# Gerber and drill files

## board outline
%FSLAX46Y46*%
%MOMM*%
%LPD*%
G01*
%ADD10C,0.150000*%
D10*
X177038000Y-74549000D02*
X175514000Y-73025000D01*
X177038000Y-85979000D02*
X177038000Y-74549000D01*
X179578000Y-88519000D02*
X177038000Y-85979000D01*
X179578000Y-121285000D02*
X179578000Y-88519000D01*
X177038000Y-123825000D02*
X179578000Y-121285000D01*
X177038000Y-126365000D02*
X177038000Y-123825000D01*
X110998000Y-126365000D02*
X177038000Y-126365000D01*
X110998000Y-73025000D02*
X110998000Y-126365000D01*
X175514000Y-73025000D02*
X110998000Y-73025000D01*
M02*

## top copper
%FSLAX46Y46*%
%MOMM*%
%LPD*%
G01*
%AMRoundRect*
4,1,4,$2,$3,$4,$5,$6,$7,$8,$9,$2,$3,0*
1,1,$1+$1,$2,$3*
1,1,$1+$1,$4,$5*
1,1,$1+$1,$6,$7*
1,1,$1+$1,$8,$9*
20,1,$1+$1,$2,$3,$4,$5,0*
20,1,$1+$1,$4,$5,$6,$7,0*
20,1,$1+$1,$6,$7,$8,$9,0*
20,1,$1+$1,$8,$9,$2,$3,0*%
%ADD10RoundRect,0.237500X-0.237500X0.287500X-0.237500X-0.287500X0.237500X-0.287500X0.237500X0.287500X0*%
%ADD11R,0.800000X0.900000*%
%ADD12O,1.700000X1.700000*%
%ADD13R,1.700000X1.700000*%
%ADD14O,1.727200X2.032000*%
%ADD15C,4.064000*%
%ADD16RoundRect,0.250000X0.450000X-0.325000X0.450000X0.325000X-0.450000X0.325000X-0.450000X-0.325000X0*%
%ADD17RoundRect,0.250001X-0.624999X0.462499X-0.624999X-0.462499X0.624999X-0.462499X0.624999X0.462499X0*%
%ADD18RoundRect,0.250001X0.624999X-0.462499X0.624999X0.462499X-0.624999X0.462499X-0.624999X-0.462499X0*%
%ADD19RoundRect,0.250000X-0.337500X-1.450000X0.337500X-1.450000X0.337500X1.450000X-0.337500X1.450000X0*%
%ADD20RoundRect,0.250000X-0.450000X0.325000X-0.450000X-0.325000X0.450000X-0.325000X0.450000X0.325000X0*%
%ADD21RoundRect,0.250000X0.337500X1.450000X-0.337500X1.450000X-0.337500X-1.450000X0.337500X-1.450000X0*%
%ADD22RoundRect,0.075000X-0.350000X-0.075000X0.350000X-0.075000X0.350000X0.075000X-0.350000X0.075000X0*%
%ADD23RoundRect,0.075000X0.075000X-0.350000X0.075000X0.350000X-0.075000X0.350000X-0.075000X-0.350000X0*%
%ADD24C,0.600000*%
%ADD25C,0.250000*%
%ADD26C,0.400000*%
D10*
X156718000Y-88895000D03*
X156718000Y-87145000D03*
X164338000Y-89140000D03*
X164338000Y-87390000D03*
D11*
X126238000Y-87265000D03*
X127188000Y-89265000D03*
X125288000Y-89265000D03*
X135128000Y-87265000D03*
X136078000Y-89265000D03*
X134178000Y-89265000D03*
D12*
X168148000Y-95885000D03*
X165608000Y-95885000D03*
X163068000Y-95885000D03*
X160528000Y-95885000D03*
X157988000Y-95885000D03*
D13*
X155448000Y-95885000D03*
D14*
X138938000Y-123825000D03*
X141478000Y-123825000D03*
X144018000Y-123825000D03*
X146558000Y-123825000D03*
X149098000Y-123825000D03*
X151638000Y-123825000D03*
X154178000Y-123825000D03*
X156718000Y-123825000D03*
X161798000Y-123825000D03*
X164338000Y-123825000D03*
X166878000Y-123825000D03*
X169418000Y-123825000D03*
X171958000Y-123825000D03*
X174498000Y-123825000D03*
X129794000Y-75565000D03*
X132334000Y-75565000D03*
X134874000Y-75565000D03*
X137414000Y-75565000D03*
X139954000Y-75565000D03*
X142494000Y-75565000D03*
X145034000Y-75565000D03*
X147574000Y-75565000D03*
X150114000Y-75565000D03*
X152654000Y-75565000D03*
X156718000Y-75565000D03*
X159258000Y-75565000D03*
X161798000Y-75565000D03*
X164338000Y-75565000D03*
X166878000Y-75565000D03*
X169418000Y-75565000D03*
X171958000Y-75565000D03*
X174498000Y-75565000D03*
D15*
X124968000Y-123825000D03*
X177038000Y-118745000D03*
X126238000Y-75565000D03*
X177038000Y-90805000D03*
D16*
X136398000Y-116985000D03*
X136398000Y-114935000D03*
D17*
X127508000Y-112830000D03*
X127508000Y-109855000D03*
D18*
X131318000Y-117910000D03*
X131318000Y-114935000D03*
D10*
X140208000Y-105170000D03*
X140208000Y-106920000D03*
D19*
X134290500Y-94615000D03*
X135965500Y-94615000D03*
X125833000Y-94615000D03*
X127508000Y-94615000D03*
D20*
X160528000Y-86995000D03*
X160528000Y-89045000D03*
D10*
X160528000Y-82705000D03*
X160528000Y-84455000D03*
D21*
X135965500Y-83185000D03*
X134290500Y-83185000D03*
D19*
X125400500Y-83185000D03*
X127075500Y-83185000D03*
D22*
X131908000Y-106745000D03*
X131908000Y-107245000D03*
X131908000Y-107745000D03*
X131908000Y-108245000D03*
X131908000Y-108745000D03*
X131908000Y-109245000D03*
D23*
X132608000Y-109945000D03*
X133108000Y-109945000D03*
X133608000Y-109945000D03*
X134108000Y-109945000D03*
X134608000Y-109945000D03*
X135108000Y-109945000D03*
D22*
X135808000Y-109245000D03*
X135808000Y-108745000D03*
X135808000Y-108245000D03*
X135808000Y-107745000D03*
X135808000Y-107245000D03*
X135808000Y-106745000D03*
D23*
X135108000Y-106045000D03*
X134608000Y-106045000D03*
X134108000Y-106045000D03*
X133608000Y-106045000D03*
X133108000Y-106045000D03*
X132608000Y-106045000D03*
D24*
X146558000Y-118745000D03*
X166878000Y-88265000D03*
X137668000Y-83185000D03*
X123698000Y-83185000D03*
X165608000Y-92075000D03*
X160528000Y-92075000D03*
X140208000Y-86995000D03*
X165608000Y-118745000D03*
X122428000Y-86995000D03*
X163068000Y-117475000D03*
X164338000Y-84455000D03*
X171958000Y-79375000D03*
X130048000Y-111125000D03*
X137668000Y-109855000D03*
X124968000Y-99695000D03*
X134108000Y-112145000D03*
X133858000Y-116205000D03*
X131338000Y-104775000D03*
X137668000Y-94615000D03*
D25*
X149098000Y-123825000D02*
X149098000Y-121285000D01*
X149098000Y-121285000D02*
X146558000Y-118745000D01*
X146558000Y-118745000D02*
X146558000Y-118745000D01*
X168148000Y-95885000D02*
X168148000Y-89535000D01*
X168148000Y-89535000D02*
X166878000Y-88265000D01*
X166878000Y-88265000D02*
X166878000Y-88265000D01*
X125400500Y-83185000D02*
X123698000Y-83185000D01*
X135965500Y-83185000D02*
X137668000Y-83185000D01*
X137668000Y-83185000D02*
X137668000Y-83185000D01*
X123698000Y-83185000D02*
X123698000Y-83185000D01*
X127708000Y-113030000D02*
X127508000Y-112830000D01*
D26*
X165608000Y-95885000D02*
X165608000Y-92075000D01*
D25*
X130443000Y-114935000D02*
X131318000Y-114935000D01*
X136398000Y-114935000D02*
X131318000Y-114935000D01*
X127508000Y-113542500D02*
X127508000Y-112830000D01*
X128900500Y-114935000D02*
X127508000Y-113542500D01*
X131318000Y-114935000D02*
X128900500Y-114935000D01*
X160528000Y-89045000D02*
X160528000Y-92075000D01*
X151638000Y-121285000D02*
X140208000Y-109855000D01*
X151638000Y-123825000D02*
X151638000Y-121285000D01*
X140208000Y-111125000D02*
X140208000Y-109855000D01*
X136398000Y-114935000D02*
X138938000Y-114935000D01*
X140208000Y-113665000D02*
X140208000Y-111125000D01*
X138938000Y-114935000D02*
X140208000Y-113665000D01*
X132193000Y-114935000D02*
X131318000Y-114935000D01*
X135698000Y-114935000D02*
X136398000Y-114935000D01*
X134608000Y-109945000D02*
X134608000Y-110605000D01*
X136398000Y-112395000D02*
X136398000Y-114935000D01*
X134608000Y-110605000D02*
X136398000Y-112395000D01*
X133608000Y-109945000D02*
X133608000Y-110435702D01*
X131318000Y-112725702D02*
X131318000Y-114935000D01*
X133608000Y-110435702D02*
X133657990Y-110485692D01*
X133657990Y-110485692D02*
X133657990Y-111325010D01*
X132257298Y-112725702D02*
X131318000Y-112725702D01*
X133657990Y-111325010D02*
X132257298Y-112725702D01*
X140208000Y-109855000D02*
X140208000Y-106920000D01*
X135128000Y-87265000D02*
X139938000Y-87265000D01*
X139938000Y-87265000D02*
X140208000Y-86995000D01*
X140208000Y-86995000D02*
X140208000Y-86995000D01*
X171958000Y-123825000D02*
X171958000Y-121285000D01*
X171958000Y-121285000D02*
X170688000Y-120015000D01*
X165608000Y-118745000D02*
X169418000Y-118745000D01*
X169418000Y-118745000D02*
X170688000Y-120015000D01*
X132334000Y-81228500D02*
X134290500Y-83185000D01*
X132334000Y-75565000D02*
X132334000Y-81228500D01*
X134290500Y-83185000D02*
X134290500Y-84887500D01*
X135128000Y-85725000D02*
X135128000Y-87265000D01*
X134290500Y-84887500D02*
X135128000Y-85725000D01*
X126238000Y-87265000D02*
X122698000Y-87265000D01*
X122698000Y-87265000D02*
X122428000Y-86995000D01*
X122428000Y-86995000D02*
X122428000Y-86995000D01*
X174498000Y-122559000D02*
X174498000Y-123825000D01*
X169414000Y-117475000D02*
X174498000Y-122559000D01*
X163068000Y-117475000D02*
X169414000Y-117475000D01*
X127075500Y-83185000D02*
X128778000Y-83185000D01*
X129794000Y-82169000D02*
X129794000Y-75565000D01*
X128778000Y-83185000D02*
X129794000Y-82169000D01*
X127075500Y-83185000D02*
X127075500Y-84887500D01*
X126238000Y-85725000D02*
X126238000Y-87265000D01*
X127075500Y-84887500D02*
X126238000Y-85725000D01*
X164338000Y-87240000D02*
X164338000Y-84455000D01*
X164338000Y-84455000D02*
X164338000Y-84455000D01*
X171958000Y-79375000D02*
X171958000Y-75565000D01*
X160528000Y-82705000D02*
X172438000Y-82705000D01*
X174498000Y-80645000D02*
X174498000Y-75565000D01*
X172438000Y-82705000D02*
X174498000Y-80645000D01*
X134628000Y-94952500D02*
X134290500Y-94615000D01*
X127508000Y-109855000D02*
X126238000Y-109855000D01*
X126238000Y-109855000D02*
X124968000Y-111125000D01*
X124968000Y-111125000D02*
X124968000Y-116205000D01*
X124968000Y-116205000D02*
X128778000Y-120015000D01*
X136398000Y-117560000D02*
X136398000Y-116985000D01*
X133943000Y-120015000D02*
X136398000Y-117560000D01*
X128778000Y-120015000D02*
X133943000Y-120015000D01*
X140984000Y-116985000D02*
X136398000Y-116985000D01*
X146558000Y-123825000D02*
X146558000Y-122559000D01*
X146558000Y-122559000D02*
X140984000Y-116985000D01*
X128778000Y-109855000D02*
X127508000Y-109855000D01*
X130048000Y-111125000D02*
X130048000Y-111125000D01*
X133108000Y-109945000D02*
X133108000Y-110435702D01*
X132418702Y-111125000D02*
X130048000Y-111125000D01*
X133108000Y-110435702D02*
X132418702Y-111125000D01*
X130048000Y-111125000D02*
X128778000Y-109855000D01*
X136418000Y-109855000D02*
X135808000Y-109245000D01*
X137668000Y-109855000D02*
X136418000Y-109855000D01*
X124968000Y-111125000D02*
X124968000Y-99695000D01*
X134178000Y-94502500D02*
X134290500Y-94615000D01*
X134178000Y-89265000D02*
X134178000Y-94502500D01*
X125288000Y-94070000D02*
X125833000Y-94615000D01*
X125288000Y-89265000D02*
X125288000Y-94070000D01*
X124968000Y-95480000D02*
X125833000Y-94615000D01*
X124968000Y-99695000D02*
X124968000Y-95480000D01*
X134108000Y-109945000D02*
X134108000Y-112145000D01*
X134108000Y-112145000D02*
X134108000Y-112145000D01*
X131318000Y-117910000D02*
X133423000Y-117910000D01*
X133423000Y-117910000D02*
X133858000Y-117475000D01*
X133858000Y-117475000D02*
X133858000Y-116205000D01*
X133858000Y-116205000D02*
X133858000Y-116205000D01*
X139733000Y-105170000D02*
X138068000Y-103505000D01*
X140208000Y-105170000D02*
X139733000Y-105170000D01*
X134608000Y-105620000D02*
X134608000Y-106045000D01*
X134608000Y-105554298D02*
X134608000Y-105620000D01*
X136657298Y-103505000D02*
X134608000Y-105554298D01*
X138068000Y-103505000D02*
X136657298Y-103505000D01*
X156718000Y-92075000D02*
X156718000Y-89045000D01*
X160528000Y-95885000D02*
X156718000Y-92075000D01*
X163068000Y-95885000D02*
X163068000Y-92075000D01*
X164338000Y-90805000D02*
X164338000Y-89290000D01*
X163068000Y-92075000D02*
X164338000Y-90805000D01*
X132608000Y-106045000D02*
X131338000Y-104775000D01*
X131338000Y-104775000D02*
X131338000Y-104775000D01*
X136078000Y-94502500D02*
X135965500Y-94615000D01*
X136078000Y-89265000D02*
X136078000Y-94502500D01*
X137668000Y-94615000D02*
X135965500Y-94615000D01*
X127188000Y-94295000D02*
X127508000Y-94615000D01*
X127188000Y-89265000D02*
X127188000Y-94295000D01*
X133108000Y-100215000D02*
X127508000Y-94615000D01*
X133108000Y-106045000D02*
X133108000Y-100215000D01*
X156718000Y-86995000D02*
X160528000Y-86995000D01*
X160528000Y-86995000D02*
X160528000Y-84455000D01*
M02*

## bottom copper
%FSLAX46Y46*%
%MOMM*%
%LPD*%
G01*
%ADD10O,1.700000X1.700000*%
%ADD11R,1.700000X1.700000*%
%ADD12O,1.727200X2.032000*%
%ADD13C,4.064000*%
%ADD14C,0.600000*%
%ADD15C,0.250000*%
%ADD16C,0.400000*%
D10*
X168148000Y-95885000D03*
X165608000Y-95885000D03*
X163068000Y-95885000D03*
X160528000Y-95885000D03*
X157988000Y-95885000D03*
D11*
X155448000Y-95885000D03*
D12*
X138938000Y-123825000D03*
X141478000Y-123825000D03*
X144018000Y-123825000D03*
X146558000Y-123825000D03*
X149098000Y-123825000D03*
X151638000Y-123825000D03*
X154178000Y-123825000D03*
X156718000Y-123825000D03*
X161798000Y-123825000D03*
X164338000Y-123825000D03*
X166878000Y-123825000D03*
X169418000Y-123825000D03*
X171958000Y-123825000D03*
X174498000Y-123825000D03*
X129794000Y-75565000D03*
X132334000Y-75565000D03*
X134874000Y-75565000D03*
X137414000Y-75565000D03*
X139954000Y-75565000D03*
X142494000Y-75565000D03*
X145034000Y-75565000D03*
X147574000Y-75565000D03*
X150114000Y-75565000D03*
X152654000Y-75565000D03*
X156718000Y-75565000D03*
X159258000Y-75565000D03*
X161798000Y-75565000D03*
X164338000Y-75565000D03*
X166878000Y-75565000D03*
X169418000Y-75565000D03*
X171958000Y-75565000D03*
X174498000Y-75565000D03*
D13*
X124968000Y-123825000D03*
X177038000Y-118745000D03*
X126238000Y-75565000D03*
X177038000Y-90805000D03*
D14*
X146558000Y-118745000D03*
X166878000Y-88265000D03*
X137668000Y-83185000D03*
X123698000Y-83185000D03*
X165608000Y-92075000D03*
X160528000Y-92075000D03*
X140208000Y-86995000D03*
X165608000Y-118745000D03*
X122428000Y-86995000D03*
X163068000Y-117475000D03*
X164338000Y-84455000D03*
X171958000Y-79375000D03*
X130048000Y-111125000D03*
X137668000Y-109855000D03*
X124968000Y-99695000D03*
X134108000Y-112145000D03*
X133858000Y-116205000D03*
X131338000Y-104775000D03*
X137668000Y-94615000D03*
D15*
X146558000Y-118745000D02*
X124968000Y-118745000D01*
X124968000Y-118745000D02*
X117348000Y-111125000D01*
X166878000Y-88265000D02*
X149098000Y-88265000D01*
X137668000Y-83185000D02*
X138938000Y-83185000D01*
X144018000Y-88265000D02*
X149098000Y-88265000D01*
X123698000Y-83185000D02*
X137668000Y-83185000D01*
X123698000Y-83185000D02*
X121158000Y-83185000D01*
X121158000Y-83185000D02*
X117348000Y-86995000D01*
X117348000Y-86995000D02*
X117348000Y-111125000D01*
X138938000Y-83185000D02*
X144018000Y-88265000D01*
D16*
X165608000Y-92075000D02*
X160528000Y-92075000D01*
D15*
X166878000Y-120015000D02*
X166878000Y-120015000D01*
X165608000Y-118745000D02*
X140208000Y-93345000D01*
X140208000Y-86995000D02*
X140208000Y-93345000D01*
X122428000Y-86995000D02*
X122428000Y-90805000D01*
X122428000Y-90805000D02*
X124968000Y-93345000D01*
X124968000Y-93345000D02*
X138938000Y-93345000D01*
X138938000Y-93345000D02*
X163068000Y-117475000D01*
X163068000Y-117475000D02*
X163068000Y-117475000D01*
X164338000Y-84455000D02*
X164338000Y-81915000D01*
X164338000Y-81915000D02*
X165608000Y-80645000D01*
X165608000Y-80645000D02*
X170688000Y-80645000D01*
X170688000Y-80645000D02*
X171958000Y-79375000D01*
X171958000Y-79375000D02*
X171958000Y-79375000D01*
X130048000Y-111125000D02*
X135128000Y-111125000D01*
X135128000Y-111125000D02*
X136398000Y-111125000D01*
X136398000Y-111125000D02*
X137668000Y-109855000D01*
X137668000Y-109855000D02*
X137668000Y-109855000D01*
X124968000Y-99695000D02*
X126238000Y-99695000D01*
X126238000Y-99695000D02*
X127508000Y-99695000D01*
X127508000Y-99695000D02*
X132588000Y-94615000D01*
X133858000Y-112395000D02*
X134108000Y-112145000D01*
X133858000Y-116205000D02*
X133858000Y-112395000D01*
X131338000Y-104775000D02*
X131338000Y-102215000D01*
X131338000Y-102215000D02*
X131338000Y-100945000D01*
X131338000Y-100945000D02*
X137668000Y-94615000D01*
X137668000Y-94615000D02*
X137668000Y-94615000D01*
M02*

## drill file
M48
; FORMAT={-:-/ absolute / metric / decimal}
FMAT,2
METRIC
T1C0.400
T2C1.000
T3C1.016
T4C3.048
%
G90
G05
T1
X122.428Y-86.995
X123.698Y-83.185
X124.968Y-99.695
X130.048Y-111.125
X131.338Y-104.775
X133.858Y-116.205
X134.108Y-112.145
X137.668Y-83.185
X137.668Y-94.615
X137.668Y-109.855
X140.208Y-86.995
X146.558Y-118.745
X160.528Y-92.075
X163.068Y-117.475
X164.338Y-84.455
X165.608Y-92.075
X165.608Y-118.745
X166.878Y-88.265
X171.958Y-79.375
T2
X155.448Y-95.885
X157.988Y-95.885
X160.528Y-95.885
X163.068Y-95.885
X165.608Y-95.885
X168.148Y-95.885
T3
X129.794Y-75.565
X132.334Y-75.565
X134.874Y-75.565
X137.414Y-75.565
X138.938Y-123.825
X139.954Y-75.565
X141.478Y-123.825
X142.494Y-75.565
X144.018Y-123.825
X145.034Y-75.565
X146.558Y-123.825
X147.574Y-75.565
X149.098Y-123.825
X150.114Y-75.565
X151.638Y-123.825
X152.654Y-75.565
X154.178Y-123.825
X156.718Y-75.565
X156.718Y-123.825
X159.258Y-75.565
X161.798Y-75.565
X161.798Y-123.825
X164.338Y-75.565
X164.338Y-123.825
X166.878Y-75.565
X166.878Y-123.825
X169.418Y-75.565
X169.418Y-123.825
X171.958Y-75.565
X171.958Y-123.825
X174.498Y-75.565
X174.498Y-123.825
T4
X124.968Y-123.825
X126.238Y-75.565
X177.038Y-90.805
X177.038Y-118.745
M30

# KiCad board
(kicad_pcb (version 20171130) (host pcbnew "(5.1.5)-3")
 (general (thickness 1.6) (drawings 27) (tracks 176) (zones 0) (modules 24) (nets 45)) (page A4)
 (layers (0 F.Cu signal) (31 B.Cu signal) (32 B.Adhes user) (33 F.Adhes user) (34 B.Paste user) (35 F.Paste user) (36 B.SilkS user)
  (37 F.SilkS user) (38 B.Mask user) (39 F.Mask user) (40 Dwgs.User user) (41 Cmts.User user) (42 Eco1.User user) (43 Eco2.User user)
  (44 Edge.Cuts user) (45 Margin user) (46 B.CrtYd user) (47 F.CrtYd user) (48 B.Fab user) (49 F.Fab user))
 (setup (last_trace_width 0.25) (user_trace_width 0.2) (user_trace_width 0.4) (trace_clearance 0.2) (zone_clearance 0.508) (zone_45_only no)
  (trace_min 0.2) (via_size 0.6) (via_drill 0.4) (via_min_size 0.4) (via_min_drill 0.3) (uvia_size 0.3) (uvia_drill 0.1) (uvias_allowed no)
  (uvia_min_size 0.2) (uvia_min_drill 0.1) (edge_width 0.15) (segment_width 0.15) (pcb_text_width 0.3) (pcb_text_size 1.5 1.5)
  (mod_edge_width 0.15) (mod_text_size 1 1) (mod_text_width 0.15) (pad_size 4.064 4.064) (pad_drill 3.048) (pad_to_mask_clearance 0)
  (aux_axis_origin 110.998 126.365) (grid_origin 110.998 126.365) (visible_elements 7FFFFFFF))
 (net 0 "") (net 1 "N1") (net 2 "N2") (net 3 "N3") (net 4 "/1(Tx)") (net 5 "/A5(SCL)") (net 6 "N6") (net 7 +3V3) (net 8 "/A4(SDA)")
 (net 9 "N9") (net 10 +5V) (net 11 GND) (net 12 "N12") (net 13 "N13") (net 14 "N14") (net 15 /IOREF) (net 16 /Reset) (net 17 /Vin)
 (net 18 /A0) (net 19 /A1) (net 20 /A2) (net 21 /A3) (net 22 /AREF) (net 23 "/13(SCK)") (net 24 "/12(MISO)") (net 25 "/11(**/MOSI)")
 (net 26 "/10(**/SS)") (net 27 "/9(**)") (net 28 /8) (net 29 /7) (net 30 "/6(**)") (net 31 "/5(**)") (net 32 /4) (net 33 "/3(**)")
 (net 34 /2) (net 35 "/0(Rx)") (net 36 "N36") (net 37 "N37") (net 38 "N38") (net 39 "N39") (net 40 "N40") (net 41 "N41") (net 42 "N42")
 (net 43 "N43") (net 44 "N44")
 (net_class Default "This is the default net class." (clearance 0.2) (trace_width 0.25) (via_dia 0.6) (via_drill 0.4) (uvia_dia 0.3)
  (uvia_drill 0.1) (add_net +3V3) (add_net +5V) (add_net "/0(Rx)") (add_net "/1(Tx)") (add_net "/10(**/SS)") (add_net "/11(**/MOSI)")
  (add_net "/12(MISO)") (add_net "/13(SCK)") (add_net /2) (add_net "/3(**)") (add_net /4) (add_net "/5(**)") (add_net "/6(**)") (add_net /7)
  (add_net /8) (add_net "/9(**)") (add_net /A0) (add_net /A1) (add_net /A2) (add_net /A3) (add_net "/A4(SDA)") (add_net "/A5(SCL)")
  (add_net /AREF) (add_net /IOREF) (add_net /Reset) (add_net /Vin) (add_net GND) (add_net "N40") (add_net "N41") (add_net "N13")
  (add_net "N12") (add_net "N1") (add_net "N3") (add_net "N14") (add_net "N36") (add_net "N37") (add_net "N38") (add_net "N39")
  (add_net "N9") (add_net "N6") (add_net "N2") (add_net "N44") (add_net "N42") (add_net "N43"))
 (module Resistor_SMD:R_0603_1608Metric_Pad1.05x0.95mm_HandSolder (layer F.Cu) (at 156.718 88.02 270)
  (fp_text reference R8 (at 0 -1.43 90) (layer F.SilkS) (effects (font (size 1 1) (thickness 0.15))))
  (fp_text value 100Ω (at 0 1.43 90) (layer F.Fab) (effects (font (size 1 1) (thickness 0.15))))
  (pad 2 smd roundrect (at 0.875 0 270) (size 1.05 0.95) (layers F.Cu F.Paste F.Mask) (roundrect_rratio 0.25) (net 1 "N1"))
  (pad 1 smd roundrect (at -0.875 0 270) (size 1.05 0.95) (layers F.Cu F.Paste F.Mask) (roundrect_rratio 0.25) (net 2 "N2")))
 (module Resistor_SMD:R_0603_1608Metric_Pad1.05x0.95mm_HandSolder (layer F.Cu) (at 164.338 88.265 270)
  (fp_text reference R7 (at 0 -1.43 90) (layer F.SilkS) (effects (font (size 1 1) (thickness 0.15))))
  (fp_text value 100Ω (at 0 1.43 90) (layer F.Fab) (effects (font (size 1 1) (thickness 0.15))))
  (pad 2 smd roundrect (at 0.875 0 270) (size 1.05 0.95) (layers F.Cu F.Paste F.Mask) (roundrect_rratio 0.25) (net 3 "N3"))
  (pad 1 smd roundrect (at -0.875 0 270) (size 1.05 0.95) (layers F.Cu F.Paste F.Mask) (roundrect_rratio 0.25) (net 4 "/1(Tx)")))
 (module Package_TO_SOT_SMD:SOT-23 (layer F.Cu) (at 126.238 88.265 90)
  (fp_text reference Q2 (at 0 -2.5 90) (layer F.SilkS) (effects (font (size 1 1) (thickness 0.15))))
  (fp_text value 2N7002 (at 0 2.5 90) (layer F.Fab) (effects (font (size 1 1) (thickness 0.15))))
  (pad 3 smd rect (at 1 0 90) (size 0.9 0.8) (layers F.Cu F.Paste F.Mask) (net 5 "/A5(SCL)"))
  (pad 2 smd rect (at -1 0.95 90) (size 0.9 0.8) (layers F.Cu F.Paste F.Mask) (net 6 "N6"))
  (pad 1 smd rect (at -1 -0.95 90) (size 0.9 0.8) (layers F.Cu F.Paste F.Mask) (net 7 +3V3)))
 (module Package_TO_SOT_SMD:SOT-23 (layer F.Cu) (at 135.128 88.265 90)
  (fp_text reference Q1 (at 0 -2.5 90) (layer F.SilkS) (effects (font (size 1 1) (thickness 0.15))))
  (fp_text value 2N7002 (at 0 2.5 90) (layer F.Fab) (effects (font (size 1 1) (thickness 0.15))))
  (pad 3 smd rect (at 1 0 90) (size 0.9 0.8) (layers F.Cu F.Paste F.Mask) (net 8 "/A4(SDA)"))
  (pad 2 smd rect (at -1 0.95 90) (size 0.9 0.8) (layers F.Cu F.Paste F.Mask) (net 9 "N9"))
  (pad 1 smd rect (at -1 -0.95 90) (size 0.9 0.8) (layers F.Cu F.Paste F.Mask) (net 7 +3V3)))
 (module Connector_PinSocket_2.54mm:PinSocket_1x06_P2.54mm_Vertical (layer F.Cu) (at 155.448 95.885 90)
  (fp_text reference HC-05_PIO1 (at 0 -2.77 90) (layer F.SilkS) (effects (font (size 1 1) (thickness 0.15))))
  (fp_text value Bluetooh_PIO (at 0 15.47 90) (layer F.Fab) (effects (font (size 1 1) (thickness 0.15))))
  (pad 6 thru_hole oval (at 0 12.7 90) (size 1.7 1.7) (drill 1) (layers *.Cu *.Mask) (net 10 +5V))
  (pad 5 thru_hole oval (at 0 10.16 90) (size 1.7 1.7) (drill 1) (layers *.Cu *.Mask) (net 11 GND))
  (pad 4 thru_hole oval (at 0 7.62 90) (size 1.7 1.7) (drill 1) (layers *.Cu *.Mask) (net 3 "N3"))
  (pad 3 thru_hole oval (at 0 5.08 90) (size 1.7 1.7) (drill 1) (layers *.Cu *.Mask) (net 1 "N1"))
  (pad 2 thru_hole oval (at 0 2.54 90) (size 1.7 1.7) (drill 1) (layers *.Cu *.Mask) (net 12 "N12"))
  (pad 1 thru_hole rect (at 0 0 90) (size 1.7 1.7) (drill 1) (layers *.Cu *.Mask) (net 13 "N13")))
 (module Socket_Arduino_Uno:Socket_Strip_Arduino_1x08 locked (layer F.Cu) (at 138.938 123.825)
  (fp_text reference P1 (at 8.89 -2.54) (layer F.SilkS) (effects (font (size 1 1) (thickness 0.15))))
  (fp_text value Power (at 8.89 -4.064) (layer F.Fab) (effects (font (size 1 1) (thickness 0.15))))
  (pad 1 thru_hole oval (at 0 0) (size 1.7272 2.032) (drill 1.016) (layers *.Cu *.Mask F.SilkS) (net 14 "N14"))
  (pad 2 thru_hole oval (at 2.54 0) (size 1.7272 2.032) (drill 1.016) (layers *.Cu *.Mask F.SilkS) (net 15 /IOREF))
  (pad 3 thru_hole oval (at 5.08 0) (size 1.7272 2.032) (drill 1.016) (layers *.Cu *.Mask F.SilkS) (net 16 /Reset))
  (pad 4 thru_hole oval (at 7.62 0) (size 1.7272 2.032) (drill 1.016) (layers *.Cu *.Mask F.SilkS) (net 7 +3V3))
  (pad 5 thru_hole oval (at 10.16 0) (size 1.7272 2.032) (drill 1.016) (layers *.Cu *.Mask F.SilkS) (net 10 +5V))
  (pad 6 thru_hole oval (at 12.7 0) (size 1.7272 2.032) (drill 1.016) (layers *.Cu *.Mask F.SilkS) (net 11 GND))
  (pad 7 thru_hole oval (at 15.24 0) (size 1.7272 2.032) (drill 1.016) (layers *.Cu *.Mask F.SilkS) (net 11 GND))
  (pad 8 thru_hole oval (at 17.78 0) (size 1.7272 2.032) (drill 1.016) (layers *.Cu *.Mask F.SilkS) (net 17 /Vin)))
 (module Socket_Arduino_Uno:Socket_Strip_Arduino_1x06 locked (layer F.Cu) (at 161.798 123.825)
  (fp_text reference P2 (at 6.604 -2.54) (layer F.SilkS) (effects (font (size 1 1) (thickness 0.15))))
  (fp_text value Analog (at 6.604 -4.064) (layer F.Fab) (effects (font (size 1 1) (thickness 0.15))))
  (pad 1 thru_hole oval (at 0 0) (size 1.7272 2.032) (drill 1.016) (layers *.Cu *.Mask F.SilkS) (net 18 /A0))
  (pad 2 thru_hole oval (at 2.54 0) (size 1.7272 2.032) (drill 1.016) (layers *.Cu *.Mask F.SilkS) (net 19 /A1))
  (pad 3 thru_hole oval (at 5.08 0) (size 1.7272 2.032) (drill 1.016) (layers *.Cu *.Mask F.SilkS) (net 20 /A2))
  (pad 4 thru_hole oval (at 7.62 0) (size 1.7272 2.032) (drill 1.016) (layers *.Cu *.Mask F.SilkS) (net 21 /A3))
  (pad 5 thru_hole oval (at 10.16 0) (size 1.7272 2.032) (drill 1.016) (layers *.Cu *.Mask F.SilkS) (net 8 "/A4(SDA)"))
  (pad 6 thru_hole oval (at 12.7 0) (size 1.7272 2.032) (drill 1.016) (layers *.Cu *.Mask F.SilkS) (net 5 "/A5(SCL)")))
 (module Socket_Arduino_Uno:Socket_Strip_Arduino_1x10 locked (layer F.Cu) (at 129.794 75.565)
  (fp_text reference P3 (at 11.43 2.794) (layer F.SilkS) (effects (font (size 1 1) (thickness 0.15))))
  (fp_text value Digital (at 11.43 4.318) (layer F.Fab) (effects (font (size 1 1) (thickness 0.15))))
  (pad 1 thru_hole oval (at 0 0) (size 1.7272 2.032) (drill 1.016) (layers *.Cu *.Mask F.SilkS) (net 5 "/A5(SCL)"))
  (pad 2 thru_hole oval (at 2.54 0) (size 1.7272 2.032) (drill 1.016) (layers *.Cu *.Mask F.SilkS) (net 8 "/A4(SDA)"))
  (pad 3 thru_hole oval (at 5.08 0) (size 1.7272 2.032) (drill 1.016) (layers *.Cu *.Mask F.SilkS) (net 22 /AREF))
  (pad 4 thru_hole oval (at 7.62 0) (size 1.7272 2.032) (drill 1.016) (layers *.Cu *.Mask F.SilkS) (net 11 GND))
  (pad 5 thru_hole oval (at 10.16 0) (size 1.7272 2.032) (drill 1.016) (layers *.Cu *.Mask F.SilkS) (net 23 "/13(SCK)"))
  (pad 6 thru_hole oval (at 12.7 0) (size 1.7272 2.032) (drill 1.016) (layers *.Cu *.Mask F.SilkS) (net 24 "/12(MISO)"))
  (pad 7 thru_hole oval (at 15.24 0) (size 1.7272 2.032) (drill 1.016) (layers *.Cu *.Mask F.SilkS) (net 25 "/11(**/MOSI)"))
  (pad 8 thru_hole oval (at 17.78 0) (size 1.7272 2.032) (drill 1.016) (layers *.Cu *.Mask F.SilkS) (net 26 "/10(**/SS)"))
  (pad 9 thru_hole oval (at 20.32 0) (size 1.7272 2.032) (drill 1.016) (layers *.Cu *.Mask F.SilkS) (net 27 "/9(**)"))
  (pad 10 thru_hole oval (at 22.86 0) (size 1.7272 2.032) (drill 1.016) (layers *.Cu *.Mask F.SilkS) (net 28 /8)))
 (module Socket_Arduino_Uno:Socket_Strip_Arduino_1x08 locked (layer F.Cu) (at 156.718 75.565)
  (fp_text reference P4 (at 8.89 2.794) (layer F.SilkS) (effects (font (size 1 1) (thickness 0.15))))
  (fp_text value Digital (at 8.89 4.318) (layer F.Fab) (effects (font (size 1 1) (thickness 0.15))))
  (pad 1 thru_hole oval (at 0 0) (size 1.7272 2.032) (drill 1.016) (layers *.Cu *.Mask F.SilkS) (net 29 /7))
  (pad 2 thru_hole oval (at 2.54 0) (size 1.7272 2.032) (drill 1.016) (layers *.Cu *.Mask F.SilkS) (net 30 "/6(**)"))
  (pad 3 thru_hole oval (at 5.08 0) (size 1.7272 2.032) (drill 1.016) (layers *.Cu *.Mask F.SilkS) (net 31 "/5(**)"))
  (pad 4 thru_hole oval (at 7.62 0) (size 1.7272 2.032) (drill 1.016) (layers *.Cu *.Mask F.SilkS) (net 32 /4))
  (pad 5 thru_hole oval (at 10.16 0) (size 1.7272 2.032) (drill 1.016) (layers *.Cu *.Mask F.SilkS) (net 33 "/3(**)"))
  (pad 6 thru_hole oval (at 12.7 0) (size 1.7272 2.032) (drill 1.016) (layers *.Cu *.Mask F.SilkS) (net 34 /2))
  (pad 7 thru_hole oval (at 15.24 0) (size 1.7272 2.032) (drill 1.016) (layers *.Cu *.Mask F.SilkS) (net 4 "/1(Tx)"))
  (pad 8 thru_hole oval (at 17.78 0) (size 1.7272 2.032) (drill 1.016) (layers *.Cu *.Mask F.SilkS) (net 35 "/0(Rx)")))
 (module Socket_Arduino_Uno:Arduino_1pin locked (layer F.Cu) (at 124.968 123.825)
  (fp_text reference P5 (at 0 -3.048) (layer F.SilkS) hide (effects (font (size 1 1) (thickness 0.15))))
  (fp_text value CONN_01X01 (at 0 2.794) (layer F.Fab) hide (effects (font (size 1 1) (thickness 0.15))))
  (pad 1 thru_hole circle (at 0 0) (size 4.064 4.064) (drill 3.048) (layers *.Cu *.Mask F.SilkS) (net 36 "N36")))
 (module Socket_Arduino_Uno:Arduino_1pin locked (layer F.Cu) (at 177.038 118.745)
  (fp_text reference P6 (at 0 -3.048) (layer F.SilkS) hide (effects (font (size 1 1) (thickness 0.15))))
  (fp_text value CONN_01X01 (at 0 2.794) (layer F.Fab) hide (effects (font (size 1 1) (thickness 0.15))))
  (pad 1 thru_hole circle (at 0 0) (size 4.064 4.064) (drill 3.048) (layers *.Cu *.Mask F.SilkS) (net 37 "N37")))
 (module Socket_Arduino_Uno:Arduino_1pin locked (layer F.Cu) (at 126.238 75.565)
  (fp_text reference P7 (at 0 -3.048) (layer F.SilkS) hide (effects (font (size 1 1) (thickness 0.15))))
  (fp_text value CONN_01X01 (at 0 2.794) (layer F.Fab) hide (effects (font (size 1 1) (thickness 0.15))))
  (pad 1 thru_hole circle (at 0 0) (size 4.064 4.064) (drill 3.048) (layers *.Cu *.Mask F.SilkS) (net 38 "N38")))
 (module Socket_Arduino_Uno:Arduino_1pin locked (layer F.Cu) (at 177.038 90.805)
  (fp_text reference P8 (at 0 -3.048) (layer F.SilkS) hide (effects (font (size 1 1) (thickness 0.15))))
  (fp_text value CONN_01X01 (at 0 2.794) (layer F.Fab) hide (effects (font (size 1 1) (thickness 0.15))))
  (pad 1 thru_hole circle (at 0 0) (size 4.064 4.064) (drill 3.048) (layers *.Cu *.Mask F.SilkS) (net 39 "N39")))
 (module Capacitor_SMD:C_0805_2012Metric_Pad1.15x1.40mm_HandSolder (layer F.Cu) (at 136.398 115.96 90)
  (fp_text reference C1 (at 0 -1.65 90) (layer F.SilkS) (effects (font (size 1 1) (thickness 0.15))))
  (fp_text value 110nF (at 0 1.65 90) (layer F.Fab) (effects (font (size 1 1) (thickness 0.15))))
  (pad 1 smd roundrect (at -1.025 0 90) (size 1.15 1.4) (layers F.Cu F.Paste F.Mask) (roundrect_rratio 0.217391) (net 7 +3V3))
  (pad 2 smd roundrect (at 1.025 0 90) (size 1.15 1.4) (layers F.Cu F.Paste F.Mask) (roundrect_rratio 0.217391) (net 11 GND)))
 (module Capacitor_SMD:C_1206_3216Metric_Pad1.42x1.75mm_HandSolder (layer F.Cu) (at 127.508 111.3425 270)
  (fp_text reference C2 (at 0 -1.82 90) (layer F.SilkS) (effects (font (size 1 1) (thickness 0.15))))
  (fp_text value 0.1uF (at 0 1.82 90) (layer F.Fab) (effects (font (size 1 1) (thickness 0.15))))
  (pad 2 smd roundrect (at 1.4875 0 270) (size 1.425 1.75) (layers F.Cu F.Paste F.Mask) (roundrect_rratio 0.175439) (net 11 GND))
  (pad 1 smd roundrect (at -1.4875 0 270) (size 1.425 1.75) (layers F.Cu F.Paste F.Mask) (roundrect_rratio 0.175439) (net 7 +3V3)))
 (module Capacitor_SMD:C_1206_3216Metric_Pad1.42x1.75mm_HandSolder (layer F.Cu) (at 131.318 116.4225 90)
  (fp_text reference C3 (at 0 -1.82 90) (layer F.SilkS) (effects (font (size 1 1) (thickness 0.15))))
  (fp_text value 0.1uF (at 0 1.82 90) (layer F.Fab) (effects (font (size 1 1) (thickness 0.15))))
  (pad 1 smd roundrect (at -1.4875 0 90) (size 1.425 1.75) (layers F.Cu F.Paste F.Mask) (roundrect_rratio 0.175439) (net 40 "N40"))
  (pad 2 smd roundrect (at 1.4875 0 90) (size 1.425 1.75) (layers F.Cu F.Paste F.Mask) (roundrect_rratio 0.175439) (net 11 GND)))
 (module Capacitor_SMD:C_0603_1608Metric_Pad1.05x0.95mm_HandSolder (layer F.Cu) (at 140.208 106.045 270)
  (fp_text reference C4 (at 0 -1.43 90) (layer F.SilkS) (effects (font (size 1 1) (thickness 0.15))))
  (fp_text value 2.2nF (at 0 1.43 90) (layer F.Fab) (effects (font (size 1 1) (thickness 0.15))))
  (pad 1 smd roundrect (at -0.875 0 270) (size 1.05 0.95) (layers F.Cu F.Paste F.Mask) (roundrect_rratio 0.25) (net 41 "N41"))
  (pad 2 smd roundrect (at 0.875 0 270) (size 1.05 0.95) (layers F.Cu F.Paste F.Mask) (roundrect_rratio 0.25) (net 11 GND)))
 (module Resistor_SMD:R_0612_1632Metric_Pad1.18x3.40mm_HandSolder (layer F.Cu) (at 135.128 94.615)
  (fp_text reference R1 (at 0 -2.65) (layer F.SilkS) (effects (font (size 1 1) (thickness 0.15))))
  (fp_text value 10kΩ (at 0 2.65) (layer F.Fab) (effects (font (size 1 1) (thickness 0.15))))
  (pad 1 smd roundrect (at -0.8375 0) (size 1.175 3.4) (layers F.Cu F.Paste F.Mask) (roundrect_rratio 0.212766) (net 7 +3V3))
  (pad 2 smd roundrect (at 0.8375 0) (size 1.175 3.4) (layers F.Cu F.Paste F.Mask) (roundrect_rratio 0.212766) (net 9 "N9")))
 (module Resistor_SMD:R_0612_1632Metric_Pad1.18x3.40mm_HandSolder (layer F.Cu) (at 126.6705 94.615)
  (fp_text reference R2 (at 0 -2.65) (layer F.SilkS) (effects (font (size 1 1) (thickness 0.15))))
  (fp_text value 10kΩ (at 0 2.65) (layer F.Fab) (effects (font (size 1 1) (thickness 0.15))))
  (pad 1 smd roundrect (at -0.8375 0) (size 1.175 3.4) (layers F.Cu F.Paste F.Mask) (roundrect_rratio 0.212766) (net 7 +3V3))
  (pad 2 smd roundrect (at 0.8375 0) (size 1.175 3.4) (layers F.Cu F.Paste F.Mask) (roundrect_rratio 0.212766) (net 6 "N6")))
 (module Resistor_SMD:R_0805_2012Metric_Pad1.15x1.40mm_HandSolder (layer F.Cu) (at 160.528 88.02 270)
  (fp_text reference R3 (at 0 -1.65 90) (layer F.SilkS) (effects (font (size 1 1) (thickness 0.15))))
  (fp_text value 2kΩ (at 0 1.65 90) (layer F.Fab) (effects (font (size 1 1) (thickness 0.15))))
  (pad 1 smd roundrect (at -1.025 0 270) (size 1.15 1.4) (layers F.Cu F.Paste F.Mask) (roundrect_rratio 0.217391) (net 2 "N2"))
  (pad 2 smd roundrect (at 1.025 0 270) (size 1.15 1.4) (layers F.Cu F.Paste F.Mask) (roundrect_rratio 0.217391) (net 11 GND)))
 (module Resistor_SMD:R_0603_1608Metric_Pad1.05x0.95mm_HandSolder (layer F.Cu) (at 160.528 83.58 270)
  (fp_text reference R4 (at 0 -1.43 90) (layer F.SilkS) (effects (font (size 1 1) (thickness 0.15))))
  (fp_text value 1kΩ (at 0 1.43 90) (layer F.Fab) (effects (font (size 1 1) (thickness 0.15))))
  (pad 1 smd roundrect (at -0.875 0 270) (size 1.05 0.95) (layers F.Cu F.Paste F.Mask) (roundrect_rratio 0.25) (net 35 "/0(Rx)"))
  (pad 2 smd roundrect (at 0.875 0 270) (size 1.05 0.95) (layers F.Cu F.Paste F.Mask) (roundrect_rratio 0.25) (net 2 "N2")))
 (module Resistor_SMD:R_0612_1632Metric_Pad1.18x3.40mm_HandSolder (layer F.Cu) (at 135.128 83.185 180)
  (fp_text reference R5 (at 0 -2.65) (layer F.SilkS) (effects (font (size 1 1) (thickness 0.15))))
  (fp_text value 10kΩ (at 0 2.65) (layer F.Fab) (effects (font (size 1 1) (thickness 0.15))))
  (pad 1 smd roundrect (at -0.8375 0 180) (size 1.175 3.4) (layers F.Cu F.Paste F.Mask) (roundrect_rratio 0.212766) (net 10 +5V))
  (pad 2 smd roundrect (at 0.8375 0 180) (size 1.175 3.4) (layers F.Cu F.Paste F.Mask) (roundrect_rratio 0.212766) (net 8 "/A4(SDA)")))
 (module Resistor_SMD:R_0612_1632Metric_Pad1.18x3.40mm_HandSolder (layer F.Cu) (at 126.238 83.185)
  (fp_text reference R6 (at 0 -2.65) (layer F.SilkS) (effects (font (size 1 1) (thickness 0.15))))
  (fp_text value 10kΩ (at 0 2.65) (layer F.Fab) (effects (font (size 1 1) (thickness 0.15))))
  (pad 1 smd roundrect (at -0.8375 0) (size 1.175 3.4) (layers F.Cu F.Paste F.Mask) (roundrect_rratio 0.212766) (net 10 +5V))
  (pad 2 smd roundrect (at 0.8375 0) (size 1.175 3.4) (layers F.Cu F.Paste F.Mask) (roundrect_rratio 0.212766) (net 5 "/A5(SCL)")))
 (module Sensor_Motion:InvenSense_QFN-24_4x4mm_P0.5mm (layer F.Cu) (at 133.858 107.995)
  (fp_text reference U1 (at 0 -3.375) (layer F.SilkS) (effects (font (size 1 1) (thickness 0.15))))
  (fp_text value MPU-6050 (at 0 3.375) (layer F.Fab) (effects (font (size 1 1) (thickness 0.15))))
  (pad 1 smd roundrect (at -1.95 -1.25) (size 0.85 0.3) (layers F.Cu F.Paste F.Mask) (roundrect_rratio 0.25) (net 11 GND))
  (pad 2 smd roundrect (at -1.95 -0.75) (size 0.85 0.3) (layers F.Cu F.Paste F.Mask) (roundrect_rratio 0.25))
  (pad 3 smd roundrect (at -1.95 -0.25) (size 0.85 0.3) (layers F.Cu F.Paste F.Mask) (roundrect_rratio 0.25))
  (pad 4 smd roundrect (at -1.95 0.25) (size 0.85 0.3) (layers F.Cu F.Paste F.Mask) (roundrect_rratio 0.25))
  (pad 5 smd roundrect (at -1.95 0.75) (size 0.85 0.3) (layers F.Cu F.Paste F.Mask) (roundrect_rratio 0.25))
  (pad 6 smd roundrect (at -1.95 1.25) (size 0.85 0.3) (layers F.Cu F.Paste F.Mask) (roundrect_rratio 0.25) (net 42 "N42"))
  (pad 7 smd roundrect (at -1.25 1.95 90) (size 0.85 0.3) (layers F.Cu F.Paste F.Mask) (roundrect_rratio 0.25) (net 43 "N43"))
  (pad 8 smd roundrect (at -0.75 1.95 90) (size 0.85 0.3) (layers F.Cu F.Paste F.Mask) (roundrect_rratio 0.25) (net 7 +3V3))
  (pad 9 smd roundrect (at -0.25 1.95 90) (size 0.85 0.3) (layers F.Cu F.Paste F.Mask) (roundrect_rratio 0.25) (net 11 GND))
  (pad 10 smd roundrect (at 0.25 1.95 90) (size 0.85 0.3) (layers F.Cu F.Paste F.Mask) (roundrect_rratio 0.25) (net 40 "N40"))
  (pad 11 smd roundrect (at 0.75 1.95 90) (size 0.85 0.3) (layers F.Cu F.Paste F.Mask) (roundrect_rratio 0.25) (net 11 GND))
  (pad 12 smd roundrect (at 1.25 1.95 90) (size 0.85 0.3) (layers F.Cu F.Paste F.Mask) (roundrect_rratio 0.25) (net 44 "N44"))
  (pad 13 smd roundrect (at 1.95 1.25) (size 0.85 0.3) (layers F.Cu F.Paste F.Mask) (roundrect_rratio 0.25) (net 7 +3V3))
  (pad 14 smd roundrect (at 1.95 0.75) (size 0.85 0.3) (layers F.Cu F.Paste F.Mask) (roundrect_rratio 0.25))
  (pad 15 smd roundrect (at 1.95 0.25) (size 0.85 0.3) (layers F.Cu F.Paste F.Mask) (roundrect_rratio 0.25))
  (pad 16 smd roundrect (at 1.95 -0.25) (size 0.85 0.3) (layers F.Cu F.Paste F.Mask) (roundrect_rratio 0.25))
  (pad 17 smd roundrect (at 1.95 -0.75) (size 0.85 0.3) (layers F.Cu F.Paste F.Mask) (roundrect_rratio 0.25))
  (pad 18 smd roundrect (at 1.95 -1.25) (size 0.85 0.3) (layers F.Cu F.Paste F.Mask) (roundrect_rratio 0.25) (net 11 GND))
  (pad 19 smd roundrect (at 1.25 -1.95 90) (size 0.85 0.3) (layers F.Cu F.Paste F.Mask) (roundrect_rratio 0.25))
  (pad 20 smd roundrect (at 0.75 -1.95 90) (size 0.85 0.3) (layers F.Cu F.Paste F.Mask) (roundrect_rratio 0.25) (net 41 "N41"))
  (pad 21 smd roundrect (at 0.25 -1.95 90) (size 0.85 0.3) (layers F.Cu F.Paste F.Mask) (roundrect_rratio 0.25))
  (pad 22 smd roundrect (at -0.25 -1.95 90) (size 0.85 0.3) (layers F.Cu F.Paste F.Mask) (roundrect_rratio 0.25))
  (pad 23 smd roundrect (at -0.75 -1.95 90) (size 0.85 0.3) (layers F.Cu F.Paste F.Mask) (roundrect_rratio 0.25) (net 6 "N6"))
  (pad 24 smd roundrect (at -1.25 -1.95 90) (size 0.85 0.3) (layers F.Cu F.Paste F.Mask) (roundrect_rratio 0.25) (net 9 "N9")))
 (gr_line (start 177.038 74.549) (end 175.514 73.025) (angle 90) (layer Edge.Cuts) (width 0.15))
 (gr_line (start 177.038 85.979) (end 177.038 74.549) (angle 90) (layer Edge.Cuts) (width 0.15))
 (gr_line (start 179.578 88.519) (end 177.038 85.979) (angle 90) (layer Edge.Cuts) (width 0.15))
 (gr_line (start 179.578 121.285) (end 179.578 88.519) (angle 90) (layer Edge.Cuts) (width 0.15))
 (gr_line (start 177.038 123.825) (end 179.578 121.285) (angle 90) (layer Edge.Cuts) (width 0.15))
 (gr_line (start 177.038 126.365) (end 177.038 123.825) (angle 90) (layer Edge.Cuts) (width 0.15))
 (gr_line (start 110.998 126.365) (end 177.038 126.365) (angle 90) (layer Edge.Cuts) (width 0.15))
 (gr_line (start 110.998 73.025) (end 110.998 126.365) (angle 90) (layer Edge.Cuts) (width 0.15))
 (gr_line (start 175.514 73.025) (end 110.998 73.025) (angle 90) (layer Edge.Cuts) (width 0.15))
 (segment (start 149.098 123.825) (end 149.098 121.285) (width 0.25) (layer F.Cu) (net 10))
 (segment (start 149.098 121.285) (end 146.558 118.745) (width 0.25) (layer F.Cu) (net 10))
 (segment (start 146.558 118.745) (end 146.558 118.745) (width 0.25) (layer F.Cu) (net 10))
 (via (at 146.558 118.745) (size 0.6) (drill 0.4) (layers F.Cu B.Cu) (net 10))
 (segment (start 146.558 118.745) (end 124.968 118.745) (width 0.25) (layer B.Cu) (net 10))
 (segment (start 124.968 118.745) (end 117.348 111.125) (width 0.25) (layer B.Cu) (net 10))
 (segment (start 168.148 95.885) (end 168.148 89.535) (width 0.25) (layer F.Cu) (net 10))
 (segment (start 168.148 89.535) (end 166.878 88.265) (width 0.25) (layer F.Cu) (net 10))
 (segment (start 166.878 88.265) (end 166.878 88.265) (width 0.25) (layer F.Cu) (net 10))
 (via (at 166.878 88.265) (size 0.6) (drill 0.4) (layers F.Cu B.Cu) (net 10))
 (segment (start 166.878 88.265) (end 149.098 88.265) (width 0.25) (layer B.Cu) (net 10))
 (segment (start 125.4005 83.185) (end 123.698 83.185) (width 0.25) (layer F.Cu) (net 10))
 (segment (start 135.9655 83.185) (end 137.668 83.185) (width 0.25) (layer F.Cu) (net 10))
 (segment (start 137.668 83.185) (end 137.668 83.185) (width 0.25) (layer F.Cu) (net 10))
 (via (at 137.668 83.185) (size 0.6) (drill 0.4) (layers F.Cu B.Cu) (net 10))
 (segment (start 137.668 83.185) (end 138.938 83.185) (width 0.25) (layer B.Cu) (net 10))
 (segment (start 144.018 88.265) (end 149.098 88.265) (width 0.25) (layer B.Cu) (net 10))
 (segment (start 123.698 83.185) (end 123.698 83.185) (width 0.25) (layer F.Cu) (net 10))
 (via (at 123.698 83.185) (size 0.6) (drill 0.4) (layers F.Cu B.Cu) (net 10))
 (segment (start 123.698 83.185) (end 137.668 83.185) (width 0.25) (layer B.Cu) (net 10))
 (segment (start 123.698 83.185) (end 121.158 83.185) (width 0.25) (layer B.Cu) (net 10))
 (segment (start 121.158 83.185) (end 117.348 86.995) (width 0.25) (layer B.Cu) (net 10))
 (segment (start 117.348 86.995) (end 117.348 111.125) (width 0.25) (layer B.Cu) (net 10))
 (segment (start 138.938 83.185) (end 144.018 88.265) (width 0.25) (layer B.Cu) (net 10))
 (segment (start 127.708 113.03) (end 127.508 112.83) (width 0.25) (layer F.Cu) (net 11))
 (via (at 165.608 92.075) (size 0.6) (drill 0.4) (layers F.Cu B.Cu) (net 11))
 (segment (start 165.608 95.885) (end 165.608 92.075) (width 0.4) (layer F.Cu) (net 11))
 (via (at 160.528 92.075) (size 0.6) (drill 0.4) (layers F.Cu B.Cu) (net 11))
 (segment (start 165.608 92.075) (end 160.528 92.075) (width 0.4) (layer B.Cu) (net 11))
 (segment (start 130.443 114.935) (end 131.318 114.935) (width 0.25) (layer F.Cu) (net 11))
 (segment (start 136.398 114.935) (end 131.318 114.935) (width 0.25) (layer F.Cu) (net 11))
 (segment (start 127.508 113.5425) (end 127.508 112.83) (width 0.25) (layer F.Cu) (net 11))
 (segment (start 128.9005 114.935) (end 127.508 113.5425) (width 0.25) (layer F.Cu) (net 11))
 (segment (start 131.318 114.935) (end 128.9005 114.935) (width 0.25) (layer F.Cu) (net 11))
 (segment (start 160.528 89.045) (end 160.528 92.075) (width 0.25) (layer F.Cu) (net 11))
 (segment (start 151.638 121.285) (end 140.208 109.855) (width 0.25) (layer F.Cu) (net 11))
 (segment (start 151.638 123.825) (end 151.638 121.285) (width 0.25) (layer F.Cu) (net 11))
 (segment (start 140.208 111.125) (end 140.208 109.855) (width 0.25) (layer F.Cu) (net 11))
 (segment (start 136.398 114.935) (end 138.938 114.935) (width 0.25) (layer F.Cu) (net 11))
 (segment (start 140.208 113.665) (end 140.208 111.125) (width 0.25) (layer F.Cu) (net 11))
 (segment (start 138.938 114.935) (end 140.208 113.665) (width 0.25) (layer F.Cu) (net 11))
 (segment (start 132.193 114.935) (end 131.318 114.935) (width 0.25) (layer F.Cu) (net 11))
 (segment (start 135.698 114.935) (end 136.398 114.935) (width 0.25) (layer F.Cu) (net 11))
 (segment (start 134.608 109.945) (end 134.608 110.605) (width 0.25) (layer F.Cu) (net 11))
 (segment (start 136.398 112.395) (end 136.398 114.935) (width 0.25) (layer F.Cu) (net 11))
 (segment (start 134.608 110.605) (end 136.398 112.395) (width 0.25) (layer F.Cu) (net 11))
 (segment (start 133.608 109.945) (end 133.608 110.435702) (width 0.25) (layer F.Cu) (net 11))
 (segment (start 131.318 112.725702) (end 131.318 114.935) (width 0.25) (layer F.Cu) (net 11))
 (segment (start 133.608 110.435702) (end 133.65799 110.485692) (width 0.25) (layer F.Cu) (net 11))
 (segment (start 133.65799 110.485692) (end 133.65799 111.32501) (width 0.25) (layer F.Cu) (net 11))
 (segment (start 132.257298 112.725702) (end 131.318 112.725702) (width 0.25) (layer F.Cu) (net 11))
 (segment (start 133.65799 111.32501) (end 132.257298 112.725702) (width 0.25) (layer F.Cu) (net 11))
 (segment (start 140.208 109.855) (end 140.208 106.92) (width 0.25) (layer F.Cu) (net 11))
 (segment (start 135.128 87.265) (end 139.938 87.265) (width 0.25) (layer F.Cu) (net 8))
 (segment (start 139.938 87.265) (end 140.208 86.995) (width 0.25) (layer F.Cu) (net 8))
 (segment (start 140.208 86.995) (end 140.208 86.995) (width 0.25) (layer F.Cu) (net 8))
 (via (at 140.208 86.995) (size 0.6) (drill 0.4) (layers F.Cu B.Cu) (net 8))
 (segment (start 166.878 120.015) (end 166.878 120.015) (width 0.25) (layer B.Cu) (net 8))
 (via (at 165.608 118.745) (size 0.6) (drill 0.4) (layers F.Cu B.Cu) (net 8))
 (segment (start 171.958 123.825) (end 171.958 121.285) (width 0.25) (layer F.Cu) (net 8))
 (segment (start 171.958 121.285) (end 170.688 120.015) (width 0.25) (layer F.Cu) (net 8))
 (segment (start 165.608 118.745) (end 140.208 93.345) (width 0.25) (layer B.Cu) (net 8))
 (segment (start 165.608 118.745) (end 169.418 118.745) (width 0.25) (layer F.Cu) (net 8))
 (segment (start 169.418 118.745) (end 170.688 120.015) (width 0.25) (layer F.Cu) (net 8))
 (segment (start 132.334 81.2285) (end 134.2905 83.185) (width 0.25) (layer F.Cu) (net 8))
 (segment (start 132.334 75.565) (end 132.334 81.2285) (width 0.25) (layer F.Cu) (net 8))
 (segment (start 134.2905 83.185) (end 134.2905 84.8875) (width 0.25) (layer F.Cu) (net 8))
 (segment (start 135.128 85.725) (end 135.128 87.265) (width 0.25) (layer F.Cu) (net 8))
 (segment (start 134.2905 84.8875) (end 135.128 85.725) (width 0.25) (layer F.Cu) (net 8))
 (segment (start 140.208 86.995) (end 140.208 93.345) (width 0.25) (layer B.Cu) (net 8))
 (segment (start 126.238 87.265) (end 122.698 87.265) (width 0.25) (layer F.Cu) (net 5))
 (segment (start 122.698 87.265) (end 122.428 86.995) (width 0.25) (layer F.Cu) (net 5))
 (segment (start 122.428 86.995) (end 122.428 86.995) (width 0.25) (layer F.Cu) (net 5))
 (via (at 122.428 86.995) (size 0.6) (drill 0.4) (layers F.Cu B.Cu) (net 5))
 (segment (start 122.428 86.995) (end 122.428 90.805) (width 0.25) (layer B.Cu) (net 5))
 (segment (start 122.428 90.805) (end 124.968 93.345) (width 0.25) (layer B.Cu) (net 5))
 (segment (start 124.968 93.345) (end 138.938 93.345) (width 0.25) (layer B.Cu) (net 5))
 (segment (start 138.938 93.345) (end 163.068 117.475) (width 0.25) (layer B.Cu) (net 5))
 (segment (start 163.068 117.475) (end 163.068 117.475) (width 0.25) (layer B.Cu) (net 5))
 (via (at 163.068 117.475) (size 0.6) (drill 0.4) (layers F.Cu B.Cu) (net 5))
 (segment (start 174.498 122.559) (end 174.498 123.825) (width 0.25) (layer F.Cu) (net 5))
 (segment (start 169.414 117.475) (end 174.498 122.559) (width 0.25) (layer F.Cu) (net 5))
 (segment (start 163.068 117.475) (end 169.414 117.475) (width 0.25) (layer F.Cu) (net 5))
 (segment (start 127.0755 83.185) (end 128.778 83.185) (width 0.25) (layer F.Cu) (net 5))
 (segment (start 129.794 82.169) (end 129.794 75.565) (width 0.25) (layer F.Cu) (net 5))
 (segment (start 128.778 83.185) (end 129.794 82.169) (width 0.25) (layer F.Cu) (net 5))
 (segment (start 127.0755 83.185) (end 127.0755 84.8875) (width 0.25) (layer F.Cu) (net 5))
 (segment (start 126.238 85.725) (end 126.238 87.265) (width 0.25) (layer F.Cu) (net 5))
 (segment (start 127.0755 84.8875) (end 126.238 85.725) (width 0.25) (layer F.Cu) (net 5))
 (segment (start 164.338 87.24) (end 164.338 84.455) (width 0.25) (layer F.Cu) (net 4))
 (segment (start 164.338 84.455) (end 164.338 84.455) (width 0.25) (layer F.Cu) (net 4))
 (via (at 164.338 84.455) (size 0.6) (drill 0.4) (layers F.Cu B.Cu) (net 4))
 (segment (start 164.338 84.455) (end 164.338 81.915) (width 0.25) (layer B.Cu) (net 4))
 (segment (start 164.338 81.915) (end 165.608 80.645) (width 0.25) (layer B.Cu) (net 4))
 (segment (start 165.608 80.645) (end 170.688 80.645) (width 0.25) (layer B.Cu) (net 4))
 (segment (start 170.688 80.645) (end 171.958 79.375) (width 0.25) (layer B.Cu) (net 4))
 (segment (start 171.958 79.375) (end 171.958 79.375) (width 0.25) (layer B.Cu) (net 4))
 (via (at 171.958 79.375) (size 0.6) (drill 0.4) (layers F.Cu B.Cu) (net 4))
 (segment (start 171.958 79.375) (end 171.958 75.565) (width 0.25) (layer F.Cu) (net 4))
 (segment (start 160.528 82.705) (end 172.438 82.705) (width 0.25) (layer F.Cu) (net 35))
 (segment (start 174.498 80.645) (end 174.498 75.565) (width 0.25) (layer F.Cu) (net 35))
 (segment (start 172.438 82.705) (end 174.498 80.645) (width 0.25) (layer F.Cu) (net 35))
 (segment (start 134.628 94.9525) (end 134.2905 94.615) (width 0.25) (layer F.Cu) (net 7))
 (segment (start 127.508 109.855) (end 126.238 109.855) (width 0.25) (layer F.Cu) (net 7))
 (segment (start 126.238 109.855) (end 124.968 111.125) (width 0.25) (layer F.Cu) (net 7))
 (segment (start 124.968 111.125) (end 124.968 116.205) (width 0.25) (layer F.Cu) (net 7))
 (segment (start 124.968 116.205) (end 128.778 120.015) (width 0.25) (layer F.Cu) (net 7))
 (segment (start 136.398 117.56) (end 136.398 116.985) (width 0.25) (layer F.Cu) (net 7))
 (segment (start 133.943 120.015) (end 136.398 117.56) (width 0.25) (layer F.Cu) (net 7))
 (segment (start 128.778 120.015) (end 133.943 120.015) (width 0.25) (layer F.Cu) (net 7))
 (segment (start 140.984 116.985) (end 136.398 116.985) (width 0.25) (layer F.Cu) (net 7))
 (segment (start 146.558 123.825) (end 146.558 122.559) (width 0.25) (layer F.Cu) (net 7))
 (segment (start 146.558 122.559) (end 140.984 116.985) (width 0.25) (layer F.Cu) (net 7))
 (segment (start 128.778 109.855) (end 127.508 109.855) (width 0.25) (layer F.Cu) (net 7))
 (segment (start 130.048 111.125) (end 130.048 111.125) (width 0.25) (layer F.Cu) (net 7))
 (segment (start 133.108 109.945) (end 133.108 110.435702) (width 0.25) (layer F.Cu) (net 7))
 (segment (start 132.418702 111.125) (end 130.048 111.125) (width 0.25) (layer F.Cu) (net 7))
 (segment (start 133.108 110.435702) (end 132.418702 111.125) (width 0.25) (layer F.Cu) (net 7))
 (segment (start 130.048 111.125) (end 128.778 109.855) (width 0.25) (layer F.Cu) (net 7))
 (via (at 130.048 111.125) (size 0.6) (drill 0.4) (layers F.Cu B.Cu) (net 7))
 (segment (start 130.048 111.125) (end 135.128 111.125) (width 0.25) (layer B.Cu) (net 7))
 (segment (start 135.128 111.125) (end 136.398 111.125) (width 0.25) (layer B.Cu) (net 7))
 (segment (start 136.398 111.125) (end 137.668 109.855) (width 0.25) (layer B.Cu) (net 7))
 (segment (start 137.668 109.855) (end 137.668 109.855) (width 0.25) (layer B.Cu) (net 7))
 (via (at 137.668 109.855) (size 0.6) (drill 0.4) (layers F.Cu B.Cu) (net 7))
 (segment (start 136.418 109.855) (end 135.808 109.245) (width 0.25) (layer F.Cu) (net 7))
 (segment (start 137.668 109.855) (end 136.418 109.855) (width 0.25) (layer F.Cu) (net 7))
 (segment (start 124.968 111.125) (end 124.968 99.695) (width 0.25) (layer F.Cu) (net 7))
 (via (at 124.968 99.695) (size 0.6) (drill 0.4) (layers F.Cu B.Cu) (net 7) (status 1000000))
 (segment (start 124.968 99.695) (end 126.238 99.695) (width 0.25) (layer B.Cu) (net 7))
 (segment (start 134.178 94.5025) (end 134.2905 94.615) (width 0.25) (layer F.Cu) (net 7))
 (segment (start 134.178 89.265) (end 134.178 94.5025) (width 0.25) (layer F.Cu) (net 7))
 (segment (start 125.288 94.07) (end 125.833 94.615) (width 0.25) (layer F.Cu) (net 7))
 (segment (start 125.288 89.265) (end 125.288 94.07) (width 0.25) (layer F.Cu) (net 7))
 (segment (start 124.968 95.48) (end 125.833 94.615) (width 0.25) (layer F.Cu) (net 7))
 (segment (start 124.968 99.695) (end 124.968 95.48) (width 0.25) (layer F.Cu) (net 7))
 (segment (start 126.238 99.695) (end 127.508 99.695) (width 0.25) (layer B.Cu) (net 7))
 (segment (start 127.508 99.695) (end 132.588 94.615) (width 0.25) (layer B.Cu) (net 7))
 (segment (start 134.108 109.945) (end 134.108 112.145) (width 0.25) (layer F.Cu) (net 40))
 (segment (start 134.108 112.145) (end 134.108 112.145) (width 0.25) (layer F.Cu) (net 40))
 (via (at 134.108 112.145) (size 0.6) (drill 0.4) (layers F.Cu B.Cu) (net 40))
 (segment (start 131.318 117.91) (end 133.423 117.91) (width 0.25) (layer F.Cu) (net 40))
 (segment (start 133.423 117.91) (end 133.858 117.475) (width 0.25) (layer F.Cu) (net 40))
 (segment (start 133.858 117.475) (end 133.858 116.205) (width 0.25) (layer F.Cu) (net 40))
 (segment (start 133.858 116.205) (end 133.858 116.205) (width 0.25) (layer F.Cu) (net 40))
 (via (at 133.858 116.205) (size 0.6) (drill 0.4) (layers F.Cu B.Cu) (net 40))
 (segment (start 133.858 112.395) (end 134.108 112.145) (width 0.25) (layer B.Cu) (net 40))
 (segment (start 133.858 116.205) (end 133.858 112.395) (width 0.25) (layer B.Cu) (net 40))
 (segment (start 139.733 105.17) (end 138.068 103.505) (width 0.25) (layer F.Cu) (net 41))
 (segment (start 140.208 105.17) (end 139.733 105.17) (width 0.25) (layer F.Cu) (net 41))
 (segment (start 134.608 105.62) (end 134.608 106.045) (width 0.25) (layer F.Cu) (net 41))
 (segment (start 134.608 105.554298) (end 134.608 105.62) (width 0.25) (layer F.Cu) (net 41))
 (segment (start 136.657298 103.505) (end 134.608 105.554298) (width 0.25) (layer F.Cu) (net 41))
 (segment (start 138.068 103.505) (end 136.657298 103.505) (width 0.25) (layer F.Cu) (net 41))
 (segment (start 156.718 92.075) (end 156.718 89.045) (width 0.25) (layer F.Cu) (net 1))
 (segment (start 160.528 95.885) (end 156.718 92.075) (width 0.25) (layer F.Cu) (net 1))
 (segment (start 163.068 95.885) (end 163.068 92.075) (width 0.25) (layer F.Cu) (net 3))
 (segment (start 164.338 90.805) (end 164.338 89.29) (width 0.25) (layer F.Cu) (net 3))
 (segment (start 163.068 92.075) (end 164.338 90.805) (width 0.25) (layer F.Cu) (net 3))
 (segment (start 132.608 106.045) (end 131.338 104.775) (width 0.25) (layer F.Cu) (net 9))
 (segment (start 131.338 104.775) (end 131.338 104.775) (width 0.25) (layer F.Cu) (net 9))
 (via (at 131.338 104.775) (size 0.6) (drill 0.4) (layers F.Cu B.Cu) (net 9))
 (segment (start 131.338 104.775) (end 131.338 102.215) (width 0.25) (layer B.Cu) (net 9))
 (segment (start 136.078 94.5025) (end 135.9655 94.615) (width 0.25) (layer F.Cu) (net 9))
 (segment (start 136.078 89.265) (end 136.078 94.5025) (width 0.25) (layer F.Cu) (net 9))
 (segment (start 131.338 102.215) (end 131.338 100.945) (width 0.25) (layer B.Cu) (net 9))
 (segment (start 131.338 100.945) (end 137.668 94.615) (width 0.25) (layer B.Cu) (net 9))
 (segment (start 137.668 94.615) (end 137.668 94.615) (width 0.25) (layer B.Cu) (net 9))
 (via (at 137.668 94.615) (size 0.6) (drill 0.4) (layers F.Cu B.Cu) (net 9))
 (segment (start 137.668 94.615) (end 135.9655 94.615) (width 0.25) (layer F.Cu) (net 9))
 (segment (start 127.188 94.295) (end 127.508 94.615) (width 0.25) (layer F.Cu) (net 6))
 (segment (start 127.188 89.265) (end 127.188 94.295) (width 0.25) (layer F.Cu) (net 6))
 (segment (start 133.108 100.215) (end 127.508 94.615) (width 0.25) (layer F.Cu) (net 6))
 (segment (start 133.108 106.045) (end 133.108 100.215) (width 0.25) (layer F.Cu) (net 6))
 (segment (start 156.718 86.995) (end 160.528 86.995) (width 0.25) (layer F.Cu) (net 2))
 (segment (start 160.528 86.995) (end 160.528 84.455) (width 0.25) (layer F.Cu) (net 2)))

